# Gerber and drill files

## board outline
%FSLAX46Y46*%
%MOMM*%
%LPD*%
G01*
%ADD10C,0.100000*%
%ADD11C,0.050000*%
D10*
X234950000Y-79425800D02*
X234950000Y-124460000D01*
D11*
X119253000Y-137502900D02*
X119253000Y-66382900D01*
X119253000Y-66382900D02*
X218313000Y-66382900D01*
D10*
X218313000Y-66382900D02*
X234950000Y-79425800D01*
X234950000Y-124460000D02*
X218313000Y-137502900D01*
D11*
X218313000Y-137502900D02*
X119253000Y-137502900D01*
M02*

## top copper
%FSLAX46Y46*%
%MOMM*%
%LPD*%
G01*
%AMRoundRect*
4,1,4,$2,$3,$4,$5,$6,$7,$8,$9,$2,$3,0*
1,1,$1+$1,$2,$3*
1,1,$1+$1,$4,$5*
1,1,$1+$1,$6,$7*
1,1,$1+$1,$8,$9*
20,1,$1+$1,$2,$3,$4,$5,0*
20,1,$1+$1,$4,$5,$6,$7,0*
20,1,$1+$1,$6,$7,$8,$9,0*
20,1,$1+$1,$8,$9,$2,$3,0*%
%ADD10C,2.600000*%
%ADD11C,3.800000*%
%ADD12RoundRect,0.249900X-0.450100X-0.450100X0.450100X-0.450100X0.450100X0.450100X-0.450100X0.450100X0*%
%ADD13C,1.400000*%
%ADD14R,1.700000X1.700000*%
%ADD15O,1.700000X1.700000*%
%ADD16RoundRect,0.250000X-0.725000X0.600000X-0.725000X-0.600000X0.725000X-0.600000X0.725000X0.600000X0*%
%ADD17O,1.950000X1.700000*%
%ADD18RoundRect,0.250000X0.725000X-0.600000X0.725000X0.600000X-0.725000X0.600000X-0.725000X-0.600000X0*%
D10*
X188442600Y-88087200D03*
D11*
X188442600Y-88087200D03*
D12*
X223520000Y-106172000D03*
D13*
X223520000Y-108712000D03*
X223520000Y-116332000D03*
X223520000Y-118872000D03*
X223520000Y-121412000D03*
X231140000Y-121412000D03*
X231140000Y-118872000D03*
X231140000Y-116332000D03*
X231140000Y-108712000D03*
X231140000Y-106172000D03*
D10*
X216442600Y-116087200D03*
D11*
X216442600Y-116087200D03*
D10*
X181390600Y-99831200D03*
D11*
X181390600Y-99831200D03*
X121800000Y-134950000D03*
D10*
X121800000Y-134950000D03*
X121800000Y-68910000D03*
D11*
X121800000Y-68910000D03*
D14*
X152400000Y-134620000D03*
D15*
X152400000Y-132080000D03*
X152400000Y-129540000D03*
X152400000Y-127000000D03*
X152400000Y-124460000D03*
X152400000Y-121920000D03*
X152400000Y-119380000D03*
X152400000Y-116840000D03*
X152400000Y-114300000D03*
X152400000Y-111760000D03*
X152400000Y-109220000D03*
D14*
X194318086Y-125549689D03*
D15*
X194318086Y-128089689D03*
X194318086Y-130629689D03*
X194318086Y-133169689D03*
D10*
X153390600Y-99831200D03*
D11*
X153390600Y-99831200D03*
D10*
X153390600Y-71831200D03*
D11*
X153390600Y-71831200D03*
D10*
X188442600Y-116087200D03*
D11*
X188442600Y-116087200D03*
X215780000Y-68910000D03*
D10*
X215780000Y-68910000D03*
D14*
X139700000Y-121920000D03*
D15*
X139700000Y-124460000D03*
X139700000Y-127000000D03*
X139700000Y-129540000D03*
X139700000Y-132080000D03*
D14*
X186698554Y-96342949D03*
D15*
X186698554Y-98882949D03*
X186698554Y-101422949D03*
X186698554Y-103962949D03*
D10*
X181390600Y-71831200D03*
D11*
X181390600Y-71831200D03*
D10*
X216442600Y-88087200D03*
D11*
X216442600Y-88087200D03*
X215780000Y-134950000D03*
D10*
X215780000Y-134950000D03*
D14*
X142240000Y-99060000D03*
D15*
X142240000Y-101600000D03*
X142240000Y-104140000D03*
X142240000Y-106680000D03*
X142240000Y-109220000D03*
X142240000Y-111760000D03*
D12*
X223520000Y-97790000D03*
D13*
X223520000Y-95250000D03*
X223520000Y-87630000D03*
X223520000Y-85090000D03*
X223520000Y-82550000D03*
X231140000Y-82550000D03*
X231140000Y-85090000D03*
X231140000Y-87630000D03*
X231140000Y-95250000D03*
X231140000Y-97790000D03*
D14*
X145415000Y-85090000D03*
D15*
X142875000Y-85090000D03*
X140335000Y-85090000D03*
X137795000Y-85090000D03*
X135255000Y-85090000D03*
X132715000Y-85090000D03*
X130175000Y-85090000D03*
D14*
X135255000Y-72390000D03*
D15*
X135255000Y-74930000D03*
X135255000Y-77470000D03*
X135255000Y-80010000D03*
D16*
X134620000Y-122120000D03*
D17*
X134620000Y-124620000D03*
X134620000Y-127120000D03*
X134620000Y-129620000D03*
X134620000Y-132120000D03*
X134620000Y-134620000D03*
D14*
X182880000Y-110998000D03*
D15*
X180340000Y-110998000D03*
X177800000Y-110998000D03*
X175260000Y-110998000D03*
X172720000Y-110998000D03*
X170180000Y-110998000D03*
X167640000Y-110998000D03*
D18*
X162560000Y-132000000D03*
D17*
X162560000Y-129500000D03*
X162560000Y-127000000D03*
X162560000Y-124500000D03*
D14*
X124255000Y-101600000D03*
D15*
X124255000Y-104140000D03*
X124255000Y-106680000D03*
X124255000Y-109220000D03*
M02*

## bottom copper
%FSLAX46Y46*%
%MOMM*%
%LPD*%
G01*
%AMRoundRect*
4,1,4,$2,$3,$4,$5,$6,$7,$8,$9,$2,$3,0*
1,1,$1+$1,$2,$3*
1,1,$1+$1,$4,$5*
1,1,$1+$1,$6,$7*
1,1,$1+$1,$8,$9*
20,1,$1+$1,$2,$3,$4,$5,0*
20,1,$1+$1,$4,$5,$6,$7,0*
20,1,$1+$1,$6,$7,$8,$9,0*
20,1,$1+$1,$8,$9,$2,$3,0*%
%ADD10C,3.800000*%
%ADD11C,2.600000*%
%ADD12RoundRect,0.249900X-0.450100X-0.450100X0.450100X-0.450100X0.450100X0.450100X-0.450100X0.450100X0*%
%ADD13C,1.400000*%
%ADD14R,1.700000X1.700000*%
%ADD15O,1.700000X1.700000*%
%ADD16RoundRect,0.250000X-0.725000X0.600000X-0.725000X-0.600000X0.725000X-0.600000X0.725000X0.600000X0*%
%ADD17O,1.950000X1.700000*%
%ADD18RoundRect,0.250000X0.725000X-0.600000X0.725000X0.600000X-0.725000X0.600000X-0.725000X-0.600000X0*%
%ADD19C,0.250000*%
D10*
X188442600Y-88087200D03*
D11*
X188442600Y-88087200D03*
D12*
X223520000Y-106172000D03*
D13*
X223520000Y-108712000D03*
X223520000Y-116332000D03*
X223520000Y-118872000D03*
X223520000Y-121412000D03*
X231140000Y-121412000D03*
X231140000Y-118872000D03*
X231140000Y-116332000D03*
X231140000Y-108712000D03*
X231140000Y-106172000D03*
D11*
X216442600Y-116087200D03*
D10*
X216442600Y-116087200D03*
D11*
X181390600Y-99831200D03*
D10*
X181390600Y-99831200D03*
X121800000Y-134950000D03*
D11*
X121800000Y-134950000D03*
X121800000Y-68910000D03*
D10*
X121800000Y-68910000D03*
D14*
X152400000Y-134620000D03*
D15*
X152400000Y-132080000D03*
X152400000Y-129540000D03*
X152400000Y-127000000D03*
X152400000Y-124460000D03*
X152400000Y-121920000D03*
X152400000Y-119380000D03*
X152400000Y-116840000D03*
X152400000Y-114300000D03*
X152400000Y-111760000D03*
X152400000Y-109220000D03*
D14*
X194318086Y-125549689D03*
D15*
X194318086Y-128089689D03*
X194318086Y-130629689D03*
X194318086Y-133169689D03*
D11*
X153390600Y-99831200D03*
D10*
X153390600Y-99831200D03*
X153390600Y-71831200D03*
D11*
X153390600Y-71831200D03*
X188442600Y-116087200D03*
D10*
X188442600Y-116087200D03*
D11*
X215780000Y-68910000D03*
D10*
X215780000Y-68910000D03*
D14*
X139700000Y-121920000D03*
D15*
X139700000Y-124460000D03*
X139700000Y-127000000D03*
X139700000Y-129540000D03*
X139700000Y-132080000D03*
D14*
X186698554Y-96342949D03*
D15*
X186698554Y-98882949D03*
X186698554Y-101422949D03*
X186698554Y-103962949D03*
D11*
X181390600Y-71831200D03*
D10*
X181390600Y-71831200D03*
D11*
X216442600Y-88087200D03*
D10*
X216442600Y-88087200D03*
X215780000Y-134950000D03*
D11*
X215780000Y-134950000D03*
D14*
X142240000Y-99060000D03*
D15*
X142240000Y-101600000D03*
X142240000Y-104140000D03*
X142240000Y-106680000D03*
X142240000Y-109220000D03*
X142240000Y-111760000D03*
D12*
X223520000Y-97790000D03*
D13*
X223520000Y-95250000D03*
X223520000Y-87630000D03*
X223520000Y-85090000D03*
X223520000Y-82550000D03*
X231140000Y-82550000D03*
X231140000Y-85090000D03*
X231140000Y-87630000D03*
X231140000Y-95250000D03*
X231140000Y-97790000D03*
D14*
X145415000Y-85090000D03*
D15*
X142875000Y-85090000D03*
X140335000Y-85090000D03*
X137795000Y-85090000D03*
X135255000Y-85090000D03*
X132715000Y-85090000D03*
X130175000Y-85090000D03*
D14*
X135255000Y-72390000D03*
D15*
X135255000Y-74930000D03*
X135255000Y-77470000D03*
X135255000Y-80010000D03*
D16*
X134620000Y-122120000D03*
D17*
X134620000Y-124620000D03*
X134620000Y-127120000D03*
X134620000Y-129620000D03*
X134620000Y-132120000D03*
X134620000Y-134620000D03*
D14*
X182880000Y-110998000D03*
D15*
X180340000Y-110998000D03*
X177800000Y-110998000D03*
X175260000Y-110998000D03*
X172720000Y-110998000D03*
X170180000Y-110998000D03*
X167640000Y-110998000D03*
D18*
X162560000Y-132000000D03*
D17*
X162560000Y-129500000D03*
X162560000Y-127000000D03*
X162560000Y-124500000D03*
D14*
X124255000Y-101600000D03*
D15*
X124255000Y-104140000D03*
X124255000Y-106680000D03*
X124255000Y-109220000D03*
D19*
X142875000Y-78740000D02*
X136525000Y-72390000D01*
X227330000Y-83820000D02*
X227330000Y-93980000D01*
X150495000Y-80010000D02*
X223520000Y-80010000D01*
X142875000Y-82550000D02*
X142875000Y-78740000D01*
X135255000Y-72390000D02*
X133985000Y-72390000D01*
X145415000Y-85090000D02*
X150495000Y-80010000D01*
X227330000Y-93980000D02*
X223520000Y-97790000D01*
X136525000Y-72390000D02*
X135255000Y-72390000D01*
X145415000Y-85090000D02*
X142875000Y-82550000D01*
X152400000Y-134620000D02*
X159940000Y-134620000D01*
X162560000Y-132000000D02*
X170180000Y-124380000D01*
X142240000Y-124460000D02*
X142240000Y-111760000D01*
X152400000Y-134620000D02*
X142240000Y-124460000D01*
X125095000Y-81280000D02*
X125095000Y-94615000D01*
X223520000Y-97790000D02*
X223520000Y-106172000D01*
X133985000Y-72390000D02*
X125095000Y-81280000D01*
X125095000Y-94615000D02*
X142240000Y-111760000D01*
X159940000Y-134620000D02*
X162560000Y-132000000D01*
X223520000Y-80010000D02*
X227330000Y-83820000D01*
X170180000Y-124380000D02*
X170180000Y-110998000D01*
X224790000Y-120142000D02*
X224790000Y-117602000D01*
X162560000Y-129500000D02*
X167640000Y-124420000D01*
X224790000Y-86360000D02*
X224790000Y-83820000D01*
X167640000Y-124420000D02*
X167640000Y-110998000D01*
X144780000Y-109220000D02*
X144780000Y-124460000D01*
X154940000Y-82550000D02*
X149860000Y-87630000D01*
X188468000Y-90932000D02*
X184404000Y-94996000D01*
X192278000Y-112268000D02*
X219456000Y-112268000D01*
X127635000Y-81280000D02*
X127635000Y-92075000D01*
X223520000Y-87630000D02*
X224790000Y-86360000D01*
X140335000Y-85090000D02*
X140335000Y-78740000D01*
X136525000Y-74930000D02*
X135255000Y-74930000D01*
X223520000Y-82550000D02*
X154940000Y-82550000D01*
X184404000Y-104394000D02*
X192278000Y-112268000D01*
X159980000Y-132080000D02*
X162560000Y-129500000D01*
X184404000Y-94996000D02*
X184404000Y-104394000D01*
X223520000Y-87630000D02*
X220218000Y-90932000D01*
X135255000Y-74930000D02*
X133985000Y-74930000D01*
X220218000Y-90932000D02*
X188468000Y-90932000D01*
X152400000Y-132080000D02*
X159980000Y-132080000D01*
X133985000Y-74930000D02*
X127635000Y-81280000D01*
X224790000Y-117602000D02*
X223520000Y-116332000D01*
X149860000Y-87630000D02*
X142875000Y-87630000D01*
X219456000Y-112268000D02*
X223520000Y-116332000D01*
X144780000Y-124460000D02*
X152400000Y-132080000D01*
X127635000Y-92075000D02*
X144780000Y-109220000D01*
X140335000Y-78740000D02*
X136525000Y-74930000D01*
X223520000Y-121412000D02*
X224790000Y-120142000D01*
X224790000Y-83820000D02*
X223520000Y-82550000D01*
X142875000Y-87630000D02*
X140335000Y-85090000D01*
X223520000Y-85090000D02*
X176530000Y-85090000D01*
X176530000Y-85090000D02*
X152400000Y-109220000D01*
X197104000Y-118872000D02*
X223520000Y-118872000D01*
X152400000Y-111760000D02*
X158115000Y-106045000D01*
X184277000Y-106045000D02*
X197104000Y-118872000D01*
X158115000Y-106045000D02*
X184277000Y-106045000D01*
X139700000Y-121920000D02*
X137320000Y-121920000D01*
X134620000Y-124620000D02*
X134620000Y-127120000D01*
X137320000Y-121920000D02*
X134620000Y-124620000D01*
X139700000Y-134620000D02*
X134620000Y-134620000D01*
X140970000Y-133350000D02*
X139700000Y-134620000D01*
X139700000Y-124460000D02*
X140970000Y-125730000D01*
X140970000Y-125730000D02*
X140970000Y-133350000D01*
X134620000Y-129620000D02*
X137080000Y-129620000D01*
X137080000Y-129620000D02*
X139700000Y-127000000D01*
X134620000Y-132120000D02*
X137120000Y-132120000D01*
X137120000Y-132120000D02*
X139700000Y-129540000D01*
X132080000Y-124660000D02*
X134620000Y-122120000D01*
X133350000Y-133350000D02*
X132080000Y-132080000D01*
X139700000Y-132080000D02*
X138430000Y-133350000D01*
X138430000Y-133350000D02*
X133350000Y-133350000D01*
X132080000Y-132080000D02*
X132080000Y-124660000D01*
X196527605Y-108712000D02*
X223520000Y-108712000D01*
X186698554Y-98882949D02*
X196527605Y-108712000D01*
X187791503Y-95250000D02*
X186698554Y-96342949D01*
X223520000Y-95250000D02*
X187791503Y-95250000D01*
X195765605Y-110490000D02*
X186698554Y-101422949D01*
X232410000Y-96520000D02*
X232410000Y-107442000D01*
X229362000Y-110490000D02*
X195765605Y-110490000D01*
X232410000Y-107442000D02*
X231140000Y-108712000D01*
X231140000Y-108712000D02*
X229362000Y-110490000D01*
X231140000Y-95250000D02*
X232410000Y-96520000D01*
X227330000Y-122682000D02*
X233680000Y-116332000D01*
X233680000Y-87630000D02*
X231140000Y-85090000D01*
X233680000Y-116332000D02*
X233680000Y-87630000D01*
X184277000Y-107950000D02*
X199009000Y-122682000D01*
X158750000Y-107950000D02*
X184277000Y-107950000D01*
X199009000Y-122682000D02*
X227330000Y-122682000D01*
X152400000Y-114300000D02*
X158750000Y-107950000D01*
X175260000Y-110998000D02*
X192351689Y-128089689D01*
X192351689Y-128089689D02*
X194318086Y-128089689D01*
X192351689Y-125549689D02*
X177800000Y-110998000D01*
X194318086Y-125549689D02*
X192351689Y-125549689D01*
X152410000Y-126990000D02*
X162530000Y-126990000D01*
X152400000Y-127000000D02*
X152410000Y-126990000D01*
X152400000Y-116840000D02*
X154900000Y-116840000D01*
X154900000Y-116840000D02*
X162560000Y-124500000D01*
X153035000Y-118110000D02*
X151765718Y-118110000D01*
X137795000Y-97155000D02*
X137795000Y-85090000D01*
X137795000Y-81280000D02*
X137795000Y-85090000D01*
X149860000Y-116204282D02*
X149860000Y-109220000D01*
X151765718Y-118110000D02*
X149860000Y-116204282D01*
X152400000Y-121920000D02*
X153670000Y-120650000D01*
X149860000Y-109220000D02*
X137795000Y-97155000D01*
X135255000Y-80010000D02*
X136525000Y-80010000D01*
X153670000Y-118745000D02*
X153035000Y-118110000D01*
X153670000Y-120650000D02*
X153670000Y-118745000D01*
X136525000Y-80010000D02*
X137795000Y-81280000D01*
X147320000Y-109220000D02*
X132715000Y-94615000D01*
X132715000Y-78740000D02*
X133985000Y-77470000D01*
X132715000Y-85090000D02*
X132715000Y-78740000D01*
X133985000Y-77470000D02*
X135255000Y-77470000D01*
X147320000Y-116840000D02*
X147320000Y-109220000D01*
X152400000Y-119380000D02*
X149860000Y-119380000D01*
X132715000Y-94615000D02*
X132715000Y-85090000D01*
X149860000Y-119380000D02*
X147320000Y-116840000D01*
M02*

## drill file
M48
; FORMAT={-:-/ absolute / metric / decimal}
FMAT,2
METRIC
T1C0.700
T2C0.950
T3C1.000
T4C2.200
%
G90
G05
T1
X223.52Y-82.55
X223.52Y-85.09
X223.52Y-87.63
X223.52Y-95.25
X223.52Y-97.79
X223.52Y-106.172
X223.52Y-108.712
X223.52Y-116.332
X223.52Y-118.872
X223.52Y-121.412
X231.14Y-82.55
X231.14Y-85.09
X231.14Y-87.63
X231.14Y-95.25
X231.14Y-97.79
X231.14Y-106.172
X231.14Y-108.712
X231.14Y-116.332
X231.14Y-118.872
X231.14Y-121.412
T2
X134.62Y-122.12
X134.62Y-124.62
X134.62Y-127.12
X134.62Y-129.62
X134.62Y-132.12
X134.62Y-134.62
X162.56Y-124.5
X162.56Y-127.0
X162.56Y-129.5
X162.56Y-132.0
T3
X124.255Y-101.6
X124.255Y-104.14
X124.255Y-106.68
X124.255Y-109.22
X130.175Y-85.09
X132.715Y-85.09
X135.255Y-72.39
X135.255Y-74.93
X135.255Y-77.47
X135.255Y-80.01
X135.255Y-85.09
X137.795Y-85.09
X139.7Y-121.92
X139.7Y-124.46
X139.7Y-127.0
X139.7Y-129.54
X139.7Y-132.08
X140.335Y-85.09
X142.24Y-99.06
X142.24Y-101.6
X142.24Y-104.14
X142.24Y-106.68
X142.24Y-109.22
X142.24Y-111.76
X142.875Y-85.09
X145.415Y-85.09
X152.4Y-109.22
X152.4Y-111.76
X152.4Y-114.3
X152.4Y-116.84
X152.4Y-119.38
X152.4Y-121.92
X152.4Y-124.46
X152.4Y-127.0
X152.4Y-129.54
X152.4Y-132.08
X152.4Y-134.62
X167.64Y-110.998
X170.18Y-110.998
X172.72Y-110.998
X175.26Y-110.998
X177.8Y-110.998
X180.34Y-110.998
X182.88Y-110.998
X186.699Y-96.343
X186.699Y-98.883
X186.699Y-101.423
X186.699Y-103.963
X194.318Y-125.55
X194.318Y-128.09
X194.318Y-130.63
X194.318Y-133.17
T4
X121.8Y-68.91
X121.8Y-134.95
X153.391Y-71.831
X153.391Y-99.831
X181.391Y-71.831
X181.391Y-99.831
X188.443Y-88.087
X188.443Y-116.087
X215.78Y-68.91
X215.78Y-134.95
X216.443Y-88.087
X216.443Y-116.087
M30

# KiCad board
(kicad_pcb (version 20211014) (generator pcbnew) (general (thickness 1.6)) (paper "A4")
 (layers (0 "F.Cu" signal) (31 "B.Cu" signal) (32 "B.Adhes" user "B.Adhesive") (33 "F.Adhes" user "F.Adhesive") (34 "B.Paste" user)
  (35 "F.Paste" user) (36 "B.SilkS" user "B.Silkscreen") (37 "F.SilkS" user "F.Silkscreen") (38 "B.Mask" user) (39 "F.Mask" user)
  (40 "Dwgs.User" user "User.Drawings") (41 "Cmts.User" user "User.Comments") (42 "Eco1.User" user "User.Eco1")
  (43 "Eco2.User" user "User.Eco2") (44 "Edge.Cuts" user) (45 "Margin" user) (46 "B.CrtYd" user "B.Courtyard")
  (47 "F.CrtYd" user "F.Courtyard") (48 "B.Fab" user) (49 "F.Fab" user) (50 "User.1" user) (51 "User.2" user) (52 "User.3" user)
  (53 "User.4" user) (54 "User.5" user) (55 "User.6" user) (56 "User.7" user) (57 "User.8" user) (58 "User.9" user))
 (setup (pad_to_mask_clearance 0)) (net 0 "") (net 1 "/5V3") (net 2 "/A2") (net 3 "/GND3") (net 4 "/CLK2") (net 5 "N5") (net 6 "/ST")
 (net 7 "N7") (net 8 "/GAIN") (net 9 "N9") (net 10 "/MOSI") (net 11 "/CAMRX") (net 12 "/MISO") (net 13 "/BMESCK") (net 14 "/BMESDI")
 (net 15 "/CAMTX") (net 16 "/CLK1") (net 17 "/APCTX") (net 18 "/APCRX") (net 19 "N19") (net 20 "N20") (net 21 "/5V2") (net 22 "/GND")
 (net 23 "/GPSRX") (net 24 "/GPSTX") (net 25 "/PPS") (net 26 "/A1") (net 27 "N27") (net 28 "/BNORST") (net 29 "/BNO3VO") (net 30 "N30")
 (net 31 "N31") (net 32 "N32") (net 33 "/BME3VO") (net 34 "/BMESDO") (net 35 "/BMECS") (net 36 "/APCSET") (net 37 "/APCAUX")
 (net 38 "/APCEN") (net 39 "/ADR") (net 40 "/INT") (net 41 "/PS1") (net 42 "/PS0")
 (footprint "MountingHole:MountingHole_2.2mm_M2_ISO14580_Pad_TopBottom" (layer "F.Cu") (at 188.4426 88.0872)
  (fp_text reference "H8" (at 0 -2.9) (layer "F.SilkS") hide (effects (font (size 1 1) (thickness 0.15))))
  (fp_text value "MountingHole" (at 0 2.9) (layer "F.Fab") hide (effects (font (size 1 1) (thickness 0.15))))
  (pad "1" connect circle (at 0 0) (size 3.8 3.8) (layers "B.Cu" "B.Mask"))
  (pad "1" thru_hole circle (at 0 0) (size 2.6 2.6) (drill 2.2) (layers *.Cu *.Mask))
  (pad "1" connect circle (at 0 0) (size 3.8 3.8) (layers "F.Cu" "F.Mask")))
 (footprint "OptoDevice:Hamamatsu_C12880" (layer "F.Cu") (at 223.52 106.172)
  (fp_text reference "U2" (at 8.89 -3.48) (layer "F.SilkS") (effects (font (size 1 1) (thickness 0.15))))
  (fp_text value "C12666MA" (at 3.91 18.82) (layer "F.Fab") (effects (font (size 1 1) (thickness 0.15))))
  (pad "1" thru_hole roundrect (at 0 0) (size 1.4 1.4) (drill 0.7) (layers *.Cu *.Mask) (roundrect_rratio 0.1785) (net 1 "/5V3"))
  (pad "2" thru_hole circle (at 0 2.54) (size 1.4 1.4) (drill 0.7) (layers *.Cu *.Mask) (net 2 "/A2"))
  (pad "3" thru_hole circle (at 0 10.16) (size 1.4 1.4) (drill 0.7) (layers *.Cu *.Mask) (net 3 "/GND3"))
  (pad "4" thru_hole circle (at 0 12.7) (size 1.4 1.4) (drill 0.7) (layers *.Cu *.Mask) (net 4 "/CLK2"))
  (pad "5" thru_hole circle (at 0 15.24) (size 1.4 1.4) (drill 0.7) (layers *.Cu *.Mask) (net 3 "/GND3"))
  (pad "6" thru_hole circle (at 7.62 15.24) (size 1.4 1.4) (drill 0.7) (layers *.Cu *.Mask) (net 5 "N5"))
  (pad "7" thru_hole circle (at 7.62 12.7) (size 1.4 1.4) (drill 0.7) (layers *.Cu *.Mask) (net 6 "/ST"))
  (pad "8" thru_hole circle (at 7.62 10.16) (size 1.4 1.4) (drill 0.7) (layers *.Cu *.Mask) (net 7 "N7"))
  (pad "9" thru_hole circle (at 7.62 2.54) (size 1.4 1.4) (drill 0.7) (layers *.Cu *.Mask) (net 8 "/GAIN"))
  (pad "10" thru_hole circle (at 7.62 0) (size 1.4 1.4) (drill 0.7) (layers *.Cu *.Mask) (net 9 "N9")))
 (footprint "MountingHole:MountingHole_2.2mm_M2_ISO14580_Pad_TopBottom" (layer "F.Cu") (at 216.4426 116.0872)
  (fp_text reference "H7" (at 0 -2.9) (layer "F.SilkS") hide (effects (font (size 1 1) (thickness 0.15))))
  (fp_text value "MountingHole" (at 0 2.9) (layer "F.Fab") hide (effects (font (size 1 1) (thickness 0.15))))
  (pad "1" thru_hole circle (at 0 0) (size 2.6 2.6) (drill 2.2) (layers *.Cu *.Mask))
  (pad "1" connect circle (at 0 0) (size 3.8 3.8) (layers "F.Cu" "F.Mask"))
  (pad "1" connect circle (at 0 0) (size 3.8 3.8) (layers "B.Cu" "B.Mask")))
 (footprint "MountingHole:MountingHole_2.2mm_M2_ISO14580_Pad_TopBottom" (layer "F.Cu") (at 181.3906 99.8312)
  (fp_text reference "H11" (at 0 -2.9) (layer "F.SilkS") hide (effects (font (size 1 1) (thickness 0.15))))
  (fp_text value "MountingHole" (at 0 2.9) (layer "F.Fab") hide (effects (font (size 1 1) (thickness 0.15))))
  (pad "1" thru_hole circle (at 0 0) (size 2.6 2.6) (drill 2.2) (layers *.Cu *.Mask))
  (pad "1" connect circle (at 0 0) (size 3.8 3.8) (layers "F.Cu" "F.Mask"))
  (pad "1" connect circle (at 0 0) (size 3.8 3.8) (layers "B.Cu" "B.Mask")))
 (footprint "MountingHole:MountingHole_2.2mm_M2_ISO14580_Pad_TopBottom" (layer "F.Cu") (at 121.8 134.95)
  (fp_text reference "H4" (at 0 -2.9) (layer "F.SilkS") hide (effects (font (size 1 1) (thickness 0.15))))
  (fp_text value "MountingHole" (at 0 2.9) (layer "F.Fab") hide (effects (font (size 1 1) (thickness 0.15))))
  (pad "1" connect circle (at 0 0) (size 3.8 3.8) (layers "F.Cu" "F.Mask"))
  (pad "1" connect circle (at 0 0) (size 3.8 3.8) (layers "B.Cu" "B.Mask"))
  (pad "1" thru_hole circle (at 0 0) (size 2.6 2.6) (drill 2.2) (layers *.Cu *.Mask)))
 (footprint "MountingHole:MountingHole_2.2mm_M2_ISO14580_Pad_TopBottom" (layer "F.Cu") (at 121.8 68.91)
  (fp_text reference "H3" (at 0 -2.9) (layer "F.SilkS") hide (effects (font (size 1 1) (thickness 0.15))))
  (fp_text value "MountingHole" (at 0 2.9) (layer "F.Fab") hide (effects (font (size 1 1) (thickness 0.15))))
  (pad "1" thru_hole circle (at 0 0) (size 2.6 2.6) (drill 2.2) (layers *.Cu *.Mask))
  (pad "1" connect circle (at 0 0) (size 3.8 3.8) (layers "B.Cu" "B.Mask"))
  (pad "1" connect circle (at 0 0) (size 3.8 3.8) (layers "F.Cu" "F.Mask")))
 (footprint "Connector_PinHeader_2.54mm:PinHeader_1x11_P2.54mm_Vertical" (layer "F.Cu") (at 152.4 134.62 180)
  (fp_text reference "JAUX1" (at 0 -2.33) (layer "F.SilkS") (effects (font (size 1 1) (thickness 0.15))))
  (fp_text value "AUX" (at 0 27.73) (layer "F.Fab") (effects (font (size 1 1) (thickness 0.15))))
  (pad "1" thru_hole rect (at 0 0 180) (size 1.7 1.7) (drill 1) (layers *.Cu *.Mask) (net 1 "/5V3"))
  (pad "2" thru_hole oval (at 0 2.54 180) (size 1.7 1.7) (drill 1) (layers *.Cu *.Mask) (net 3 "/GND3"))
  (pad "3" thru_hole oval (at 0 5.08 180) (size 1.7 1.7) (drill 1) (layers *.Cu *.Mask) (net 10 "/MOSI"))
  (pad "4" thru_hole oval (at 0 7.62 180) (size 1.7 1.7) (drill 1) (layers *.Cu *.Mask) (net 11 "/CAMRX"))
  (pad "5" thru_hole oval (at 0 10.16 180) (size 1.7 1.7) (drill 1) (layers *.Cu *.Mask) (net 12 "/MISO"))
  (pad "6" thru_hole oval (at 0 12.7 180) (size 1.7 1.7) (drill 1) (layers *.Cu *.Mask) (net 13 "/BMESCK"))
  (pad "7" thru_hole oval (at 0 15.24 180) (size 1.7 1.7) (drill 1) (layers *.Cu *.Mask) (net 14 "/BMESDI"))
  (pad "8" thru_hole oval (at 0 17.78 180) (size 1.7 1.7) (drill 1) (layers *.Cu *.Mask) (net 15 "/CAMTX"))
  (pad "9" thru_hole oval (at 0 20.32 180) (size 1.7 1.7) (drill 1) (layers *.Cu *.Mask) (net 6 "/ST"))
  (pad "10" thru_hole oval (at 0 22.86 180) (size 1.7 1.7) (drill 1) (layers *.Cu *.Mask) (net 4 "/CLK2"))
  (pad "11" thru_hole oval (at 0 25.4 180) (size 1.7 1.7) (drill 1) (layers *.Cu *.Mask) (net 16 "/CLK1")))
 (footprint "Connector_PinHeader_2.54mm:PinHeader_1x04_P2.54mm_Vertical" (layer "F.Cu") (at 194.318086 125.549689)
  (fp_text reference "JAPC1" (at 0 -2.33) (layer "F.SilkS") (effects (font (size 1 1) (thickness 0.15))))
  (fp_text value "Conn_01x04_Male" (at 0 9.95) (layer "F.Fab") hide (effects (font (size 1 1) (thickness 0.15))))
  (pad "1" thru_hole rect (at 0 0) (size 1.7 1.7) (drill 1) (layers *.Cu *.Mask) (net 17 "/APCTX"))
  (pad "2" thru_hole oval (at 0 2.54) (size 1.7 1.7) (drill 1) (layers *.Cu *.Mask) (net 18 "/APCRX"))
  (pad "3" thru_hole oval (at 0 5.08) (size 1.7 1.7) (drill 1) (layers *.Cu *.Mask) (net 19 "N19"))
  (pad "4" thru_hole oval (at 0 7.62) (size 1.7 1.7) (drill 1) (layers *.Cu *.Mask) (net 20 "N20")))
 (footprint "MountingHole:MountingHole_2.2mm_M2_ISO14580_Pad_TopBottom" (layer "F.Cu") (at 153.3906 99.8312)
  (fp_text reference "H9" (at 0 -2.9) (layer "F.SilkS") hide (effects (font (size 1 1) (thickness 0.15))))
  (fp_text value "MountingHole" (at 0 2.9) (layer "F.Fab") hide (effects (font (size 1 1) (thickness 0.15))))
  (pad "1" thru_hole circle (at 0 0) (size 2.6 2.6) (drill 2.2) (layers *.Cu *.Mask))
  (pad "1" connect circle (at 0 0) (size 3.8 3.8) (layers "F.Cu" "F.Mask"))
  (pad "1" connect circle (at 0 0) (size 3.8 3.8) (layers "B.Cu" "B.Mask")))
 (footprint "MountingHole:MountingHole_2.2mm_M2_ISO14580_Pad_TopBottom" (layer "F.Cu") (at 153.3906 71.8312)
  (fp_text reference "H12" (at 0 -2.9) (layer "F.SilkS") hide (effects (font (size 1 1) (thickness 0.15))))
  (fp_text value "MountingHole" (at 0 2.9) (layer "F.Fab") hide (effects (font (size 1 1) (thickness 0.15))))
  (pad "1" connect circle (at 0 0) (size 3.8 3.8) (layers "B.Cu" "B.Mask"))
  (pad "1" thru_hole circle (at 0 0) (size 2.6 2.6) (drill 2.2) (layers *.Cu *.Mask))
  (pad "1" connect circle (at 0 0) (size 3.8 3.8) (layers "F.Cu" "F.Mask")))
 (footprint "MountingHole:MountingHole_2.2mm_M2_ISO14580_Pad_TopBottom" (layer "F.Cu") (at 188.4426 116.0872)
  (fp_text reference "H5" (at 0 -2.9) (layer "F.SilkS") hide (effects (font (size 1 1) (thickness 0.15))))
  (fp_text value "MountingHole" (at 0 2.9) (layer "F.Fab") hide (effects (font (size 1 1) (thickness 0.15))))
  (pad "1" thru_hole circle (at 0 0) (size 2.6 2.6) (drill 2.2) (layers *.Cu *.Mask))
  (pad "1" connect circle (at 0 0) (size 3.8 3.8) (layers "F.Cu" "F.Mask"))
  (pad "1" connect circle (at 0 0) (size 3.8 3.8) (layers "B.Cu" "B.Mask")))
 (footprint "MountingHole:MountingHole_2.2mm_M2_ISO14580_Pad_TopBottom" (layer "F.Cu") (at 215.78 68.91)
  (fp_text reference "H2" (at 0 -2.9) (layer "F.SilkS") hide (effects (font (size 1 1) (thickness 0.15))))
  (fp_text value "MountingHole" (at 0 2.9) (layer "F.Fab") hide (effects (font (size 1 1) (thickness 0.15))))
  (pad "1" connect circle (at 0 0) (size 3.8 3.8) (layers "F.Cu" "F.Mask"))
  (pad "1" thru_hole circle (at 0 0) (size 2.6 2.6) (drill 2.2) (layers *.Cu *.Mask))
  (pad "1" connect circle (at 0 0) (size 3.8 3.8) (layers "B.Cu" "B.Mask")))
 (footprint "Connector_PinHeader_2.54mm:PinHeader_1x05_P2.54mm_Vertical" (layer "F.Cu") (at 139.7 121.92)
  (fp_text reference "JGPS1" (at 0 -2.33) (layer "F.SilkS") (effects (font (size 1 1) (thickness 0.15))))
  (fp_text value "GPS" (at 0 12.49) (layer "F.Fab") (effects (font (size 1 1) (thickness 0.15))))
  (pad "1" thru_hole rect (at 0 0) (size 1.7 1.7) (drill 1) (layers *.Cu *.Mask) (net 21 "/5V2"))
  (pad "2" thru_hole oval (at 0 2.54) (size 1.7 1.7) (drill 1) (layers *.Cu *.Mask) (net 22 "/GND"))
  (pad "3" thru_hole oval (at 0 5.08) (size 1.7 1.7) (drill 1) (layers *.Cu *.Mask) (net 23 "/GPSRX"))
  (pad "4" thru_hole oval (at 0 7.62) (size 1.7 1.7) (drill 1) (layers *.Cu *.Mask) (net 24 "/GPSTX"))
  (pad "5" thru_hole oval (at 0 10.16) (size 1.7 1.7) (drill 1) (layers *.Cu *.Mask) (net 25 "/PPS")))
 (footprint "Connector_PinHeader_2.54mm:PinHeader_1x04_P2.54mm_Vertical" (layer "F.Cu") (at 186.698554 96.342949)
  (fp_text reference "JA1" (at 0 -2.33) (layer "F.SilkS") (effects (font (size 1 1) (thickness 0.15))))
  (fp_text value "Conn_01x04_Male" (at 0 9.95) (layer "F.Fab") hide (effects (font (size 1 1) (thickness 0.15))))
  (pad "1" thru_hole rect (at 0 0) (size 1.7 1.7) (drill 1) (layers *.Cu *.Mask) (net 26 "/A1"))
  (pad "2" thru_hole oval (at 0 2.54) (size 1.7 1.7) (drill 1) (layers *.Cu *.Mask) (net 2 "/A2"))
  (pad "3" thru_hole oval (at 0 5.08) (size 1.7 1.7) (drill 1) (layers *.Cu *.Mask) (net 8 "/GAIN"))
  (pad "4" thru_hole oval (at 0 7.62) (size 1.7 1.7) (drill 1) (layers *.Cu *.Mask) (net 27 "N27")))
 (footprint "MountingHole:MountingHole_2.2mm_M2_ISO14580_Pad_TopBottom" (layer "F.Cu") (at 181.3906 71.8312)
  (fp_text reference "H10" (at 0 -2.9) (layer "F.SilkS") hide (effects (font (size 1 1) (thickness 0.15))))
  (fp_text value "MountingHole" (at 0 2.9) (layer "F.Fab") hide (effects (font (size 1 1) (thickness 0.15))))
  (pad "1" thru_hole circle (at 0 0) (size 2.6 2.6) (drill 2.2) (layers *.Cu *.Mask))
  (pad "1" connect circle (at 0 0) (size 3.8 3.8) (layers "F.Cu" "F.Mask"))
  (pad "1" connect circle (at 0 0) (size 3.8 3.8) (layers "B.Cu" "B.Mask")))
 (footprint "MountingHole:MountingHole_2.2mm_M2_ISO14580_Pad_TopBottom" (layer "F.Cu") (at 216.4426 88.0872)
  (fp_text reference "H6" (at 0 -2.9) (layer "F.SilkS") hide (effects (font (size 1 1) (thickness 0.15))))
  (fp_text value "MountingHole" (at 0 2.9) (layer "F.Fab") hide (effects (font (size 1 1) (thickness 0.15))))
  (pad "1" thru_hole circle (at 0 0) (size 2.6 2.6) (drill 2.2) (layers *.Cu *.Mask))
  (pad "1" connect circle (at 0 0) (size 3.8 3.8) (layers "F.Cu" "F.Mask"))
  (pad "1" connect circle (at 0 0) (size 3.8 3.8) (layers "B.Cu" "B.Mask")))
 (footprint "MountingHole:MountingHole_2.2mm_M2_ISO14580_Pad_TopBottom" (layer "F.Cu") (at 215.78 134.95)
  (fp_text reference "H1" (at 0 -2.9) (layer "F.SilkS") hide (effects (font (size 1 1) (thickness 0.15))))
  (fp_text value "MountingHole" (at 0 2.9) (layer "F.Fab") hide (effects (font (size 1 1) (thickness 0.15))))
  (pad "1" connect circle (at 0 0) (size 3.8 3.8) (layers "B.Cu" "B.Mask"))
  (pad "1" connect circle (at 0 0) (size 3.8 3.8) (layers "F.Cu" "F.Mask"))
  (pad "1" thru_hole circle (at 0 0) (size 2.6 2.6) (drill 2.2) (layers *.Cu *.Mask)))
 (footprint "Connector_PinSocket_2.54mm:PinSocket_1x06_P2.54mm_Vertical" (layer "B.Cu") (at 142.24 99.06 180)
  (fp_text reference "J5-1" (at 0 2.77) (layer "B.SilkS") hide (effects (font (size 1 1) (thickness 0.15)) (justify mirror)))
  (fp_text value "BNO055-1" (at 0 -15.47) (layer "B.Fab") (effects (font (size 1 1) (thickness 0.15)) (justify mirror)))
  (pad "1" thru_hole rect (at 0 0 180) (size 1.7 1.7) (drill 1) (layers *.Cu *.Mask) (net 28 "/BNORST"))
  (pad "2" thru_hole oval (at 0 -2.54 180) (size 1.7 1.7) (drill 1) (layers *.Cu *.Mask) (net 13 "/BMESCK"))
  (pad "3" thru_hole oval (at 0 -5.08 180) (size 1.7 1.7) (drill 1) (layers *.Cu *.Mask) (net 14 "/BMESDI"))
  (pad "4" thru_hole oval (at 0 -7.62 180) (size 1.7 1.7) (drill 1) (layers *.Cu *.Mask) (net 3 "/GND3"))
  (pad "5" thru_hole oval (at 0 -10.16 180) (size 1.7 1.7) (drill 1) (layers *.Cu *.Mask) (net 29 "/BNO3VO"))
  (pad "6" thru_hole oval (at 0 -12.7 180) (size 1.7 1.7) (drill 1) (layers *.Cu *.Mask) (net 1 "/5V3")))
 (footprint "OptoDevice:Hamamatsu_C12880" (layer "B.Cu") (at 223.52 97.79)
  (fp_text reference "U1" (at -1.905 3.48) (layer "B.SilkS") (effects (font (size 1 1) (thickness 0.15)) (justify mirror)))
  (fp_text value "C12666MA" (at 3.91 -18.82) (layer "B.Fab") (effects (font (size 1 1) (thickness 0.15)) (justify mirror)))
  (pad "1" thru_hole roundrect (at 0 0) (size 1.4 1.4) (drill 0.7) (layers *.Cu *.Mask) (roundrect_rratio 0.1785) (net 1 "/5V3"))
  (pad "2" thru_hole circle (at 0 -2.54) (size 1.4 1.4) (drill 0.7) (layers *.Cu *.Mask) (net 26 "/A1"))
  (pad "3" thru_hole circle (at 0 -10.16) (size 1.4 1.4) (drill 0.7) (layers *.Cu *.Mask) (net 3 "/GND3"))
  (pad "4" thru_hole circle (at 0 -12.7) (size 1.4 1.4) (drill 0.7) (layers *.Cu *.Mask) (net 16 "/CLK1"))
  (pad "5" thru_hole circle (at 0 -15.24) (size 1.4 1.4) (drill 0.7) (layers *.Cu *.Mask) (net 3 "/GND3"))
  (pad "6" thru_hole circle (at 7.62 -15.24) (size 1.4 1.4) (drill 0.7) (layers *.Cu *.Mask) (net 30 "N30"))
  (pad "7" thru_hole circle (at 7.62 -12.7) (size 1.4 1.4) (drill 0.7) (layers *.Cu *.Mask) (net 6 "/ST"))
  (pad "8" thru_hole circle (at 7.62 -10.16) (size 1.4 1.4) (drill 0.7) (layers *.Cu *.Mask) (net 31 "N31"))
  (pad "9" thru_hole circle (at 7.62 -2.54) (size 1.4 1.4) (drill 0.7) (layers *.Cu *.Mask) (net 8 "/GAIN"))
  (pad "10" thru_hole circle (at 7.62 0) (size 1.4 1.4) (drill 0.7) (layers *.Cu *.Mask) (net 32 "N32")))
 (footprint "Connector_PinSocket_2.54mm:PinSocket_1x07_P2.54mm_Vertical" (layer "B.Cu") (at 145.415 85.09 90)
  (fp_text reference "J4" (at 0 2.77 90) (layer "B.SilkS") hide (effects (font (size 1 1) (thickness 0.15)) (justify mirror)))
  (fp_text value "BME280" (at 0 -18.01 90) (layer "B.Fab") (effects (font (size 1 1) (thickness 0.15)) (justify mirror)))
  (pad "1" thru_hole rect (at 0 0 90) (size 1.7 1.7) (drill 1) (layers *.Cu *.Mask) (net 1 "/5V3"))
  (pad "2" thru_hole oval (at 0 -2.54 90) (size 1.7 1.7) (drill 1) (layers *.Cu *.Mask) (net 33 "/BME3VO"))
  (pad "3" thru_hole oval (at 0 -5.08 90) (size 1.7 1.7) (drill 1) (layers *.Cu *.Mask) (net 3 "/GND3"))
  (pad "4" thru_hole oval (at 0 -7.62 90) (size 1.7 1.7) (drill 1) (layers *.Cu *.Mask) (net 13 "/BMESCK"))
  (pad "5" thru_hole oval (at 0 -10.16 90) (size 1.7 1.7) (drill 1) (layers *.Cu *.Mask) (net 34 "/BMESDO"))
  (pad "6" thru_hole oval (at 0 -12.7 90) (size 1.7 1.7) (drill 1) (layers *.Cu *.Mask) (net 14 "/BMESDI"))
  (pad "7" thru_hole oval (at 0 -15.24 90) (size 1.7 1.7) (drill 1) (layers *.Cu *.Mask) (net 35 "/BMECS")))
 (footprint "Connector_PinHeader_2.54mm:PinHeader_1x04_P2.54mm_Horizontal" (layer "B.Cu") (at 135.255 72.39 180)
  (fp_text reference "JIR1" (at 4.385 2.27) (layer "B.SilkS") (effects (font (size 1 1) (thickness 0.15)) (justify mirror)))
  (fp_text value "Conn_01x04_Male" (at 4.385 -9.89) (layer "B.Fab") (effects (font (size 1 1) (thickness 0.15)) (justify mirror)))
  (pad "1" thru_hole rect (at 0 0 180) (size 1.7 1.7) (drill 1) (layers *.Cu *.Mask) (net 1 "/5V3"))
  (pad "2" thru_hole oval (at 0 -2.54 180) (size 1.7 1.7) (drill 1) (layers *.Cu *.Mask) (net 3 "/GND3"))
  (pad "3" thru_hole oval (at 0 -5.08 180) (size 1.7 1.7) (drill 1) (layers *.Cu *.Mask) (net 14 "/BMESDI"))
  (pad "4" thru_hole oval (at 0 -7.62 180) (size 1.7 1.7) (drill 1) (layers *.Cu *.Mask) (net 13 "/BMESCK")))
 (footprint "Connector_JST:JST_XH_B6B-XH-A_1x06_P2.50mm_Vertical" (layer "B.Cu") (at 134.62 122.12 -90)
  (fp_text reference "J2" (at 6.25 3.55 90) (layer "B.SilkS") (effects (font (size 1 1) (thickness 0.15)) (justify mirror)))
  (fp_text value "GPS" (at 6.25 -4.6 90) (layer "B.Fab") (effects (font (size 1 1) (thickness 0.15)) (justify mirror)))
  (pad "1" thru_hole roundrect (at 0 0 270) (size 1.7 1.95) (drill 0.95) (layers *.Cu *.Mask) (roundrect_rratio 0.147059) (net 25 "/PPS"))
  (pad "2" thru_hole oval (at 2.5 0 270) (size 1.7 1.95) (drill 0.95) (layers *.Cu *.Mask) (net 21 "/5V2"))
  (pad "3" thru_hole oval (at 5 0 270) (size 1.7 1.95) (drill 0.95) (layers *.Cu *.Mask) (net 21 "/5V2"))
  (pad "4" thru_hole oval (at 7.5 0 270) (size 1.7 1.95) (drill 0.95) (layers *.Cu *.Mask) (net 23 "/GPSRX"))
  (pad "5" thru_hole oval (at 10 0 270) (size 1.7 1.95) (drill 0.95) (layers *.Cu *.Mask) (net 24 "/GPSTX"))
  (pad "6" thru_hole oval (at 12.5 0 270) (size 1.7 1.95) (drill 0.95) (layers *.Cu *.Mask) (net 22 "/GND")))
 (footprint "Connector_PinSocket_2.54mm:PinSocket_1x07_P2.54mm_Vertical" (layer "B.Cu") (at 182.88 110.998 90)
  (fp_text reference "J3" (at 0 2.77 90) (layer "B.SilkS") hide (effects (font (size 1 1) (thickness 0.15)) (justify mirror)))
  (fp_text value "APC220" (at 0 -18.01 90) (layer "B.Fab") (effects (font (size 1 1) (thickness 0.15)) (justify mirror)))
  (pad "1" thru_hole rect (at 0 0 90) (size 1.7 1.7) (drill 1) (layers *.Cu *.Mask) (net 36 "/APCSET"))
  (pad "2" thru_hole oval (at 0 -2.54 90) (size 1.7 1.7) (drill 1) (layers *.Cu *.Mask) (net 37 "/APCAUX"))
  (pad "3" thru_hole oval (at 0 -5.08 90) (size 1.7 1.7) (drill 1) (layers *.Cu *.Mask) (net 17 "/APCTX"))
  (pad "4" thru_hole oval (at 0 -7.62 90) (size 1.7 1.7) (drill 1) (layers *.Cu *.Mask) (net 18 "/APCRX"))
  (pad "5" thru_hole oval (at 0 -10.16 90) (size 1.7 1.7) (drill 1) (layers *.Cu *.Mask) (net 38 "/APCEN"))
  (pad "6" thru_hole oval (at 0 -12.7 90) (size 1.7 1.7) (drill 1) (layers *.Cu *.Mask) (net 1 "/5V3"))
  (pad "7" thru_hole oval (at 0 -15.24 90) (size 1.7 1.7) (drill 1) (layers *.Cu *.Mask) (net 3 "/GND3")))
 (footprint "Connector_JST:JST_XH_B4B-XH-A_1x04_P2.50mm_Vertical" (layer "B.Cu") (at 162.56 132 90)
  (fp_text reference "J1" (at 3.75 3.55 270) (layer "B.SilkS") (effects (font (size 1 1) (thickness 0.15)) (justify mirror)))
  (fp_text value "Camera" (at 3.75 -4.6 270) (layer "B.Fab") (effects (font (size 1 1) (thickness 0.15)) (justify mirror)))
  (pad "1" thru_hole roundrect (at 0 0 90) (size 1.7 1.95) (drill 0.95) (layers *.Cu *.Mask) (roundrect_rratio 0.147059) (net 1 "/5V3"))
  (pad "2" thru_hole oval (at 2.5 0 90) (size 1.7 1.95) (drill 0.95) (layers *.Cu *.Mask) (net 3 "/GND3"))
  (pad "3" thru_hole oval (at 5 0 90) (size 1.7 1.95) (drill 0.95) (layers *.Cu *.Mask) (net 11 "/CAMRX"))
  (pad "4" thru_hole oval (at 7.5 0 90) (size 1.7 1.95) (drill 0.95) (layers *.Cu *.Mask) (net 15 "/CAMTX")))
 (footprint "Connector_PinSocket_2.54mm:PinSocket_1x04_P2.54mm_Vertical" (layer "B.Cu") (at 124.255 101.6 180)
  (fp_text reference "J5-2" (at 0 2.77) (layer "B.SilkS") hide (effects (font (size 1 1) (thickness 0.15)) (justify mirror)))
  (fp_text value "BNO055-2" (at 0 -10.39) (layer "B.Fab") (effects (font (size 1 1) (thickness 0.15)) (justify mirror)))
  (pad "1" thru_hole rect (at 0 0 180) (size 1.7 1.7) (drill 1) (layers *.Cu *.Mask) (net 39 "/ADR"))
  (pad "2" thru_hole oval (at 0 -2.54 180) (size 1.7 1.7) (drill 1) (layers *.Cu *.Mask) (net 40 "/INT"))
  (pad "3" thru_hole oval (at 0 -5.08 180) (size 1.7 1.7) (drill 1) (layers *.Cu *.Mask) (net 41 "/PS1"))
  (pad "4" thru_hole oval (at 0 -7.62 180) (size 1.7 1.7) (drill 1) (layers *.Cu *.Mask) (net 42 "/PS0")))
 (gr_line (start 234.95 79.4258) (end 234.95 124.46) (layer "Edge.Cuts") (width 0.1))
 (gr_line (start 119.253 137.5029) (end 119.253 66.3829) (layer "Edge.Cuts") (width 0.05))
 (gr_line (start 119.253 66.3829) (end 218.313 66.3829) (layer "Edge.Cuts") (width 0.05))
 (gr_line (start 218.313 66.3829) (end 234.95 79.4258) (layer "Edge.Cuts") (width 0.1))
 (gr_line (start 234.95 124.46) (end 218.313 137.5029) (layer "Edge.Cuts") (width 0.1))
 (gr_line (start 218.313 137.5029) (end 119.253 137.5029) (layer "Edge.Cuts") (width 0.05))
 (segment (start 142.875 78.74) (end 136.525 72.39) (width 0.25) (layer "B.Cu") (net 1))
 (segment (start 227.33 83.82) (end 227.33 93.98) (width 0.25) (layer "B.Cu") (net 1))
 (segment (start 150.495 80.01) (end 223.52 80.01) (width 0.25) (layer "B.Cu") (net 1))
 (segment (start 142.875 82.55) (end 142.875 78.74) (width 0.25) (layer "B.Cu") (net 1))
 (segment (start 135.255 72.39) (end 133.985 72.39) (width 0.25) (layer "B.Cu") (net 1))
 (segment (start 145.415 85.09) (end 150.495 80.01) (width 0.25) (layer "B.Cu") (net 1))
 (segment (start 227.33 93.98) (end 223.52 97.79) (width 0.25) (layer "B.Cu") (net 1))
 (segment (start 136.525 72.39) (end 135.255 72.39) (width 0.25) (layer "B.Cu") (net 1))
 (segment (start 145.415 85.09) (end 142.875 82.55) (width 0.25) (layer "B.Cu") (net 1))
 (segment (start 152.4 134.62) (end 159.94 134.62) (width 0.25) (layer "B.Cu") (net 1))
 (segment (start 162.56 132) (end 170.18 124.38) (width 0.25) (layer "B.Cu") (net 1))
 (segment (start 142.24 124.46) (end 142.24 111.76) (width 0.25) (layer "B.Cu") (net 1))
 (segment (start 152.4 134.62) (end 142.24 124.46) (width 0.25) (layer "B.Cu") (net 1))
 (segment (start 125.095 81.28) (end 125.095 94.615) (width 0.25) (layer "B.Cu") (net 1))
 (segment (start 223.52 97.79) (end 223.52 106.172) (width 0.25) (layer "B.Cu") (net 1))
 (segment (start 133.985 72.39) (end 125.095 81.28) (width 0.25) (layer "B.Cu") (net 1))
 (segment (start 125.095 94.615) (end 142.24 111.76) (width 0.25) (layer "B.Cu") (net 1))
 (segment (start 159.94 134.62) (end 162.56 132) (width 0.25) (layer "B.Cu") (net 1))
 (segment (start 223.52 80.01) (end 227.33 83.82) (width 0.25) (layer "B.Cu") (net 1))
 (segment (start 170.18 124.38) (end 170.18 110.998) (width 0.25) (layer "B.Cu") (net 1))
 (segment (start 224.79 120.142) (end 224.79 117.602) (width 0.25) (layer "B.Cu") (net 3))
 (segment (start 162.56 129.5) (end 167.64 124.42) (width 0.25) (layer "B.Cu") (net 3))
 (segment (start 224.79 86.36) (end 224.79 83.82) (width 0.25) (layer "B.Cu") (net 3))
 (segment (start 167.64 124.42) (end 167.64 110.998) (width 0.25) (layer "B.Cu") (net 3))
 (segment (start 144.78 109.22) (end 144.78 124.46) (width 0.25) (layer "B.Cu") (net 3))
 (segment (start 154.94 82.55) (end 149.86 87.63) (width 0.25) (layer "B.Cu") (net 3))
 (segment (start 188.468 90.932) (end 184.404 94.996) (width 0.25) (layer "B.Cu") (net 3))
 (segment (start 192.278 112.268) (end 219.456 112.268) (width 0.25) (layer "B.Cu") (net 3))
 (segment (start 127.635 81.28) (end 127.635 92.075) (width 0.25) (layer "B.Cu") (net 3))
 (segment (start 223.52 87.63) (end 224.79 86.36) (width 0.25) (layer "B.Cu") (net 3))
 (segment (start 140.335 85.09) (end 140.335 78.74) (width 0.25) (layer "B.Cu") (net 3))
 (segment (start 136.525 74.93) (end 135.255 74.93) (width 0.25) (layer "B.Cu") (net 3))
 (segment (start 223.52 82.55) (end 154.94 82.55) (width 0.25) (layer "B.Cu") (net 3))
 (segment (start 184.404 104.394) (end 192.278 112.268) (width 0.25) (layer "B.Cu") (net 3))
 (segment (start 159.98 132.08) (end 162.56 129.5) (width 0.25) (layer "B.Cu") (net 3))
 (segment (start 184.404 94.996) (end 184.404 104.394) (width 0.25) (layer "B.Cu") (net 3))
 (segment (start 223.52 87.63) (end 220.218 90.932) (width 0.25) (layer "B.Cu") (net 3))
 (segment (start 135.255 74.93) (end 133.985 74.93) (width 0.25) (layer "B.Cu") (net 3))
 (segment (start 220.218 90.932) (end 188.468 90.932) (width 0.25) (layer "B.Cu") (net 3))
 (segment (start 152.4 132.08) (end 159.98 132.08) (width 0.25) (layer "B.Cu") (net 3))
 (segment (start 133.985 74.93) (end 127.635 81.28) (width 0.25) (layer "B.Cu") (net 3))
 (segment (start 224.79 117.602) (end 223.52 116.332) (width 0.25) (layer "B.Cu") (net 3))
 (segment (start 149.86 87.63) (end 142.875 87.63) (width 0.25) (layer "B.Cu") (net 3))
 (segment (start 219.456 112.268) (end 223.52 116.332) (width 0.25) (layer "B.Cu") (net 3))
 (segment (start 144.78 124.46) (end 152.4 132.08) (width 0.25) (layer "B.Cu") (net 3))
 (segment (start 127.635 92.075) (end 144.78 109.22) (width 0.25) (layer "B.Cu") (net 3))
 (segment (start 140.335 78.74) (end 136.525 74.93) (width 0.25) (layer "B.Cu") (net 3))
 (segment (start 223.52 121.412) (end 224.79 120.142) (width 0.25) (layer "B.Cu") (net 3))
 (segment (start 224.79 83.82) (end 223.52 82.55) (width 0.25) (layer "B.Cu") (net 3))
 (segment (start 142.875 87.63) (end 140.335 85.09) (width 0.25) (layer "B.Cu") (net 3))
 (segment (start 223.52 85.09) (end 176.53 85.09) (width 0.25) (layer "B.Cu") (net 16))
 (segment (start 176.53 85.09) (end 152.4 109.22) (width 0.25) (layer "B.Cu") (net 16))
 (segment (start 197.104 118.872) (end 223.52 118.872) (width 0.25) (layer "B.Cu") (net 4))
 (segment (start 152.4 111.76) (end 158.115 106.045) (width 0.25) (layer "B.Cu") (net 4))
 (segment (start 184.277 106.045) (end 197.104 118.872) (width 0.25) (layer "B.Cu") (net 4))
 (segment (start 158.115 106.045) (end 184.277 106.045) (width 0.25) (layer "B.Cu") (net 4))
 (segment (start 139.7 121.92) (end 137.32 121.92) (width 0.25) (layer "B.Cu") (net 21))
 (segment (start 134.62 124.62) (end 134.62 127.12) (width 0.25) (layer "B.Cu") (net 21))
 (segment (start 137.32 121.92) (end 134.62 124.62) (width 0.25) (layer "B.Cu") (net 21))
 (segment (start 139.7 134.62) (end 134.62 134.62) (width 0.25) (layer "B.Cu") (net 22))
 (segment (start 140.97 133.35) (end 139.7 134.62) (width 0.25) (layer "B.Cu") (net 22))
 (segment (start 139.7 124.46) (end 140.97 125.73) (width 0.25) (layer "B.Cu") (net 22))
 (segment (start 140.97 125.73) (end 140.97 133.35) (width 0.25) (layer "B.Cu") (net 22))
 (segment (start 134.62 129.62) (end 137.08 129.62) (width 0.25) (layer "B.Cu") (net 23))
 (segment (start 137.08 129.62) (end 139.7 127) (width 0.25) (layer "B.Cu") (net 23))
 (segment (start 134.62 132.12) (end 137.12 132.12) (width 0.25) (layer "B.Cu") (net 24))
 (segment (start 137.12 132.12) (end 139.7 129.54) (width 0.25) (layer "B.Cu") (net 24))
 (segment (start 132.08 124.66) (end 134.62 122.12) (width 0.25) (layer "B.Cu") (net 25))
 (segment (start 133.35 133.35) (end 132.08 132.08) (width 0.25) (layer "B.Cu") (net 25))
 (segment (start 139.7 132.08) (end 138.43 133.35) (width 0.25) (layer "B.Cu") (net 25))
 (segment (start 138.43 133.35) (end 133.35 133.35) (width 0.25) (layer "B.Cu") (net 25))
 (segment (start 132.08 132.08) (end 132.08 124.66) (width 0.25) (layer "B.Cu") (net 25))
 (segment (start 196.527605 108.712) (end 223.52 108.712) (width 0.25) (layer "B.Cu") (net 2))
 (segment (start 186.698554 98.882949) (end 196.527605 108.712) (width 0.25) (layer "B.Cu") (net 2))
 (segment (start 187.791503 95.25) (end 186.698554 96.342949) (width 0.25) (layer "B.Cu") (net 26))
 (segment (start 223.52 95.25) (end 187.791503 95.25) (width 0.25) (layer "B.Cu") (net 26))
 (segment (start 195.765605 110.49) (end 186.698554 101.422949) (width 0.25) (layer "B.Cu") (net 8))
 (segment (start 232.41 96.52) (end 232.41 107.442) (width 0.25) (layer "B.Cu") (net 8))
 (segment (start 229.362 110.49) (end 195.765605 110.49) (width 0.25) (layer "B.Cu") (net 8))
 (segment (start 232.41 107.442) (end 231.14 108.712) (width 0.25) (layer "B.Cu") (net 8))
 (segment (start 231.14 108.712) (end 229.362 110.49) (width 0.25) (layer "B.Cu") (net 8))
 (segment (start 231.14 95.25) (end 232.41 96.52) (width 0.25) (layer "B.Cu") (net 8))
 (segment (start 227.33 122.682) (end 233.68 116.332) (width 0.25) (layer "B.Cu") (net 6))
 (segment (start 233.68 87.63) (end 231.14 85.09) (width 0.25) (layer "B.Cu") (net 6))
 (segment (start 233.68 116.332) (end 233.68 87.63) (width 0.25) (layer "B.Cu") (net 6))
 (segment (start 184.277 107.95) (end 199.009 122.682) (width 0.25) (layer "B.Cu") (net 6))
 (segment (start 158.75 107.95) (end 184.277 107.95) (width 0.25) (layer "B.Cu") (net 6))
 (segment (start 199.009 122.682) (end 227.33 122.682) (width 0.25) (layer "B.Cu") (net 6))
 (segment (start 152.4 114.3) (end 158.75 107.95) (width 0.25) (layer "B.Cu") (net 6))
 (segment (start 175.26 110.998) (end 192.351689 128.089689) (width 0.25) (layer "B.Cu") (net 18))
 (segment (start 192.351689 128.089689) (end 194.318086 128.089689) (width 0.25) (layer "B.Cu") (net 18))
 (segment (start 192.351689 125.549689) (end 177.8 110.998) (width 0.25) (layer "B.Cu") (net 17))
 (segment (start 194.318086 125.549689) (end 192.351689 125.549689) (width 0.25) (layer "B.Cu") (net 17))
 (segment (start 152.41 126.99) (end 162.53 126.99) (width 0.25) (layer "B.Cu") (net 11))
 (segment (start 152.4 127) (end 152.41 126.99) (width 0.25) (layer "B.Cu") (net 11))
 (segment (start 152.4 116.84) (end 154.9 116.84) (width 0.25) (layer "B.Cu") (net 15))
 (segment (start 154.9 116.84) (end 162.56 124.5) (width 0.25) (layer "B.Cu") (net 15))
 (segment (start 153.035 118.11) (end 151.765718 118.11) (width 0.25) (layer "B.Cu") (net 13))
 (segment (start 137.795 97.155) (end 137.795 85.09) (width 0.25) (layer "B.Cu") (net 13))
 (segment (start 137.795 81.28) (end 137.795 85.09) (width 0.25) (layer "B.Cu") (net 13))
 (segment (start 149.86 116.204282) (end 149.86 109.22) (width 0.25) (layer "B.Cu") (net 13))
 (segment (start 151.765718 118.11) (end 149.86 116.204282) (width 0.25) (layer "B.Cu") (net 13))
 (segment (start 152.4 121.92) (end 153.67 120.65) (width 0.25) (layer "B.Cu") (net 13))
 (segment (start 149.86 109.22) (end 137.795 97.155) (width 0.25) (layer "B.Cu") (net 13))
 (segment (start 135.255 80.01) (end 136.525 80.01) (width 0.25) (layer "B.Cu") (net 13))
 (segment (start 153.67 118.745) (end 153.035 118.11) (width 0.25) (layer "B.Cu") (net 13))
 (segment (start 153.67 120.65) (end 153.67 118.745) (width 0.25) (layer "B.Cu") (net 13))
 (segment (start 136.525 80.01) (end 137.795 81.28) (width 0.25) (layer "B.Cu") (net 13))
 (segment (start 147.32 109.22) (end 132.715 94.615) (width 0.25) (layer "B.Cu") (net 14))
 (segment (start 132.715 78.74) (end 133.985 77.47) (width 0.25) (layer "B.Cu") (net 14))
 (segment (start 132.715 85.09) (end 132.715 78.74) (width 0.25) (layer "B.Cu") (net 14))
 (segment (start 133.985 77.47) (end 135.255 77.47) (width 0.25) (layer "B.Cu") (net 14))
 (segment (start 147.32 116.84) (end 147.32 109.22) (width 0.25) (layer "B.Cu") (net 14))
 (segment (start 152.4 119.38) (end 149.86 119.38) (width 0.25) (layer "B.Cu") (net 14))
 (segment (start 132.715 94.615) (end 132.715 85.09) (width 0.25) (layer "B.Cu") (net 14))
 (segment (start 149.86 119.38) (end 147.32 116.84) (width 0.25) (layer "B.Cu") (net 14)))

